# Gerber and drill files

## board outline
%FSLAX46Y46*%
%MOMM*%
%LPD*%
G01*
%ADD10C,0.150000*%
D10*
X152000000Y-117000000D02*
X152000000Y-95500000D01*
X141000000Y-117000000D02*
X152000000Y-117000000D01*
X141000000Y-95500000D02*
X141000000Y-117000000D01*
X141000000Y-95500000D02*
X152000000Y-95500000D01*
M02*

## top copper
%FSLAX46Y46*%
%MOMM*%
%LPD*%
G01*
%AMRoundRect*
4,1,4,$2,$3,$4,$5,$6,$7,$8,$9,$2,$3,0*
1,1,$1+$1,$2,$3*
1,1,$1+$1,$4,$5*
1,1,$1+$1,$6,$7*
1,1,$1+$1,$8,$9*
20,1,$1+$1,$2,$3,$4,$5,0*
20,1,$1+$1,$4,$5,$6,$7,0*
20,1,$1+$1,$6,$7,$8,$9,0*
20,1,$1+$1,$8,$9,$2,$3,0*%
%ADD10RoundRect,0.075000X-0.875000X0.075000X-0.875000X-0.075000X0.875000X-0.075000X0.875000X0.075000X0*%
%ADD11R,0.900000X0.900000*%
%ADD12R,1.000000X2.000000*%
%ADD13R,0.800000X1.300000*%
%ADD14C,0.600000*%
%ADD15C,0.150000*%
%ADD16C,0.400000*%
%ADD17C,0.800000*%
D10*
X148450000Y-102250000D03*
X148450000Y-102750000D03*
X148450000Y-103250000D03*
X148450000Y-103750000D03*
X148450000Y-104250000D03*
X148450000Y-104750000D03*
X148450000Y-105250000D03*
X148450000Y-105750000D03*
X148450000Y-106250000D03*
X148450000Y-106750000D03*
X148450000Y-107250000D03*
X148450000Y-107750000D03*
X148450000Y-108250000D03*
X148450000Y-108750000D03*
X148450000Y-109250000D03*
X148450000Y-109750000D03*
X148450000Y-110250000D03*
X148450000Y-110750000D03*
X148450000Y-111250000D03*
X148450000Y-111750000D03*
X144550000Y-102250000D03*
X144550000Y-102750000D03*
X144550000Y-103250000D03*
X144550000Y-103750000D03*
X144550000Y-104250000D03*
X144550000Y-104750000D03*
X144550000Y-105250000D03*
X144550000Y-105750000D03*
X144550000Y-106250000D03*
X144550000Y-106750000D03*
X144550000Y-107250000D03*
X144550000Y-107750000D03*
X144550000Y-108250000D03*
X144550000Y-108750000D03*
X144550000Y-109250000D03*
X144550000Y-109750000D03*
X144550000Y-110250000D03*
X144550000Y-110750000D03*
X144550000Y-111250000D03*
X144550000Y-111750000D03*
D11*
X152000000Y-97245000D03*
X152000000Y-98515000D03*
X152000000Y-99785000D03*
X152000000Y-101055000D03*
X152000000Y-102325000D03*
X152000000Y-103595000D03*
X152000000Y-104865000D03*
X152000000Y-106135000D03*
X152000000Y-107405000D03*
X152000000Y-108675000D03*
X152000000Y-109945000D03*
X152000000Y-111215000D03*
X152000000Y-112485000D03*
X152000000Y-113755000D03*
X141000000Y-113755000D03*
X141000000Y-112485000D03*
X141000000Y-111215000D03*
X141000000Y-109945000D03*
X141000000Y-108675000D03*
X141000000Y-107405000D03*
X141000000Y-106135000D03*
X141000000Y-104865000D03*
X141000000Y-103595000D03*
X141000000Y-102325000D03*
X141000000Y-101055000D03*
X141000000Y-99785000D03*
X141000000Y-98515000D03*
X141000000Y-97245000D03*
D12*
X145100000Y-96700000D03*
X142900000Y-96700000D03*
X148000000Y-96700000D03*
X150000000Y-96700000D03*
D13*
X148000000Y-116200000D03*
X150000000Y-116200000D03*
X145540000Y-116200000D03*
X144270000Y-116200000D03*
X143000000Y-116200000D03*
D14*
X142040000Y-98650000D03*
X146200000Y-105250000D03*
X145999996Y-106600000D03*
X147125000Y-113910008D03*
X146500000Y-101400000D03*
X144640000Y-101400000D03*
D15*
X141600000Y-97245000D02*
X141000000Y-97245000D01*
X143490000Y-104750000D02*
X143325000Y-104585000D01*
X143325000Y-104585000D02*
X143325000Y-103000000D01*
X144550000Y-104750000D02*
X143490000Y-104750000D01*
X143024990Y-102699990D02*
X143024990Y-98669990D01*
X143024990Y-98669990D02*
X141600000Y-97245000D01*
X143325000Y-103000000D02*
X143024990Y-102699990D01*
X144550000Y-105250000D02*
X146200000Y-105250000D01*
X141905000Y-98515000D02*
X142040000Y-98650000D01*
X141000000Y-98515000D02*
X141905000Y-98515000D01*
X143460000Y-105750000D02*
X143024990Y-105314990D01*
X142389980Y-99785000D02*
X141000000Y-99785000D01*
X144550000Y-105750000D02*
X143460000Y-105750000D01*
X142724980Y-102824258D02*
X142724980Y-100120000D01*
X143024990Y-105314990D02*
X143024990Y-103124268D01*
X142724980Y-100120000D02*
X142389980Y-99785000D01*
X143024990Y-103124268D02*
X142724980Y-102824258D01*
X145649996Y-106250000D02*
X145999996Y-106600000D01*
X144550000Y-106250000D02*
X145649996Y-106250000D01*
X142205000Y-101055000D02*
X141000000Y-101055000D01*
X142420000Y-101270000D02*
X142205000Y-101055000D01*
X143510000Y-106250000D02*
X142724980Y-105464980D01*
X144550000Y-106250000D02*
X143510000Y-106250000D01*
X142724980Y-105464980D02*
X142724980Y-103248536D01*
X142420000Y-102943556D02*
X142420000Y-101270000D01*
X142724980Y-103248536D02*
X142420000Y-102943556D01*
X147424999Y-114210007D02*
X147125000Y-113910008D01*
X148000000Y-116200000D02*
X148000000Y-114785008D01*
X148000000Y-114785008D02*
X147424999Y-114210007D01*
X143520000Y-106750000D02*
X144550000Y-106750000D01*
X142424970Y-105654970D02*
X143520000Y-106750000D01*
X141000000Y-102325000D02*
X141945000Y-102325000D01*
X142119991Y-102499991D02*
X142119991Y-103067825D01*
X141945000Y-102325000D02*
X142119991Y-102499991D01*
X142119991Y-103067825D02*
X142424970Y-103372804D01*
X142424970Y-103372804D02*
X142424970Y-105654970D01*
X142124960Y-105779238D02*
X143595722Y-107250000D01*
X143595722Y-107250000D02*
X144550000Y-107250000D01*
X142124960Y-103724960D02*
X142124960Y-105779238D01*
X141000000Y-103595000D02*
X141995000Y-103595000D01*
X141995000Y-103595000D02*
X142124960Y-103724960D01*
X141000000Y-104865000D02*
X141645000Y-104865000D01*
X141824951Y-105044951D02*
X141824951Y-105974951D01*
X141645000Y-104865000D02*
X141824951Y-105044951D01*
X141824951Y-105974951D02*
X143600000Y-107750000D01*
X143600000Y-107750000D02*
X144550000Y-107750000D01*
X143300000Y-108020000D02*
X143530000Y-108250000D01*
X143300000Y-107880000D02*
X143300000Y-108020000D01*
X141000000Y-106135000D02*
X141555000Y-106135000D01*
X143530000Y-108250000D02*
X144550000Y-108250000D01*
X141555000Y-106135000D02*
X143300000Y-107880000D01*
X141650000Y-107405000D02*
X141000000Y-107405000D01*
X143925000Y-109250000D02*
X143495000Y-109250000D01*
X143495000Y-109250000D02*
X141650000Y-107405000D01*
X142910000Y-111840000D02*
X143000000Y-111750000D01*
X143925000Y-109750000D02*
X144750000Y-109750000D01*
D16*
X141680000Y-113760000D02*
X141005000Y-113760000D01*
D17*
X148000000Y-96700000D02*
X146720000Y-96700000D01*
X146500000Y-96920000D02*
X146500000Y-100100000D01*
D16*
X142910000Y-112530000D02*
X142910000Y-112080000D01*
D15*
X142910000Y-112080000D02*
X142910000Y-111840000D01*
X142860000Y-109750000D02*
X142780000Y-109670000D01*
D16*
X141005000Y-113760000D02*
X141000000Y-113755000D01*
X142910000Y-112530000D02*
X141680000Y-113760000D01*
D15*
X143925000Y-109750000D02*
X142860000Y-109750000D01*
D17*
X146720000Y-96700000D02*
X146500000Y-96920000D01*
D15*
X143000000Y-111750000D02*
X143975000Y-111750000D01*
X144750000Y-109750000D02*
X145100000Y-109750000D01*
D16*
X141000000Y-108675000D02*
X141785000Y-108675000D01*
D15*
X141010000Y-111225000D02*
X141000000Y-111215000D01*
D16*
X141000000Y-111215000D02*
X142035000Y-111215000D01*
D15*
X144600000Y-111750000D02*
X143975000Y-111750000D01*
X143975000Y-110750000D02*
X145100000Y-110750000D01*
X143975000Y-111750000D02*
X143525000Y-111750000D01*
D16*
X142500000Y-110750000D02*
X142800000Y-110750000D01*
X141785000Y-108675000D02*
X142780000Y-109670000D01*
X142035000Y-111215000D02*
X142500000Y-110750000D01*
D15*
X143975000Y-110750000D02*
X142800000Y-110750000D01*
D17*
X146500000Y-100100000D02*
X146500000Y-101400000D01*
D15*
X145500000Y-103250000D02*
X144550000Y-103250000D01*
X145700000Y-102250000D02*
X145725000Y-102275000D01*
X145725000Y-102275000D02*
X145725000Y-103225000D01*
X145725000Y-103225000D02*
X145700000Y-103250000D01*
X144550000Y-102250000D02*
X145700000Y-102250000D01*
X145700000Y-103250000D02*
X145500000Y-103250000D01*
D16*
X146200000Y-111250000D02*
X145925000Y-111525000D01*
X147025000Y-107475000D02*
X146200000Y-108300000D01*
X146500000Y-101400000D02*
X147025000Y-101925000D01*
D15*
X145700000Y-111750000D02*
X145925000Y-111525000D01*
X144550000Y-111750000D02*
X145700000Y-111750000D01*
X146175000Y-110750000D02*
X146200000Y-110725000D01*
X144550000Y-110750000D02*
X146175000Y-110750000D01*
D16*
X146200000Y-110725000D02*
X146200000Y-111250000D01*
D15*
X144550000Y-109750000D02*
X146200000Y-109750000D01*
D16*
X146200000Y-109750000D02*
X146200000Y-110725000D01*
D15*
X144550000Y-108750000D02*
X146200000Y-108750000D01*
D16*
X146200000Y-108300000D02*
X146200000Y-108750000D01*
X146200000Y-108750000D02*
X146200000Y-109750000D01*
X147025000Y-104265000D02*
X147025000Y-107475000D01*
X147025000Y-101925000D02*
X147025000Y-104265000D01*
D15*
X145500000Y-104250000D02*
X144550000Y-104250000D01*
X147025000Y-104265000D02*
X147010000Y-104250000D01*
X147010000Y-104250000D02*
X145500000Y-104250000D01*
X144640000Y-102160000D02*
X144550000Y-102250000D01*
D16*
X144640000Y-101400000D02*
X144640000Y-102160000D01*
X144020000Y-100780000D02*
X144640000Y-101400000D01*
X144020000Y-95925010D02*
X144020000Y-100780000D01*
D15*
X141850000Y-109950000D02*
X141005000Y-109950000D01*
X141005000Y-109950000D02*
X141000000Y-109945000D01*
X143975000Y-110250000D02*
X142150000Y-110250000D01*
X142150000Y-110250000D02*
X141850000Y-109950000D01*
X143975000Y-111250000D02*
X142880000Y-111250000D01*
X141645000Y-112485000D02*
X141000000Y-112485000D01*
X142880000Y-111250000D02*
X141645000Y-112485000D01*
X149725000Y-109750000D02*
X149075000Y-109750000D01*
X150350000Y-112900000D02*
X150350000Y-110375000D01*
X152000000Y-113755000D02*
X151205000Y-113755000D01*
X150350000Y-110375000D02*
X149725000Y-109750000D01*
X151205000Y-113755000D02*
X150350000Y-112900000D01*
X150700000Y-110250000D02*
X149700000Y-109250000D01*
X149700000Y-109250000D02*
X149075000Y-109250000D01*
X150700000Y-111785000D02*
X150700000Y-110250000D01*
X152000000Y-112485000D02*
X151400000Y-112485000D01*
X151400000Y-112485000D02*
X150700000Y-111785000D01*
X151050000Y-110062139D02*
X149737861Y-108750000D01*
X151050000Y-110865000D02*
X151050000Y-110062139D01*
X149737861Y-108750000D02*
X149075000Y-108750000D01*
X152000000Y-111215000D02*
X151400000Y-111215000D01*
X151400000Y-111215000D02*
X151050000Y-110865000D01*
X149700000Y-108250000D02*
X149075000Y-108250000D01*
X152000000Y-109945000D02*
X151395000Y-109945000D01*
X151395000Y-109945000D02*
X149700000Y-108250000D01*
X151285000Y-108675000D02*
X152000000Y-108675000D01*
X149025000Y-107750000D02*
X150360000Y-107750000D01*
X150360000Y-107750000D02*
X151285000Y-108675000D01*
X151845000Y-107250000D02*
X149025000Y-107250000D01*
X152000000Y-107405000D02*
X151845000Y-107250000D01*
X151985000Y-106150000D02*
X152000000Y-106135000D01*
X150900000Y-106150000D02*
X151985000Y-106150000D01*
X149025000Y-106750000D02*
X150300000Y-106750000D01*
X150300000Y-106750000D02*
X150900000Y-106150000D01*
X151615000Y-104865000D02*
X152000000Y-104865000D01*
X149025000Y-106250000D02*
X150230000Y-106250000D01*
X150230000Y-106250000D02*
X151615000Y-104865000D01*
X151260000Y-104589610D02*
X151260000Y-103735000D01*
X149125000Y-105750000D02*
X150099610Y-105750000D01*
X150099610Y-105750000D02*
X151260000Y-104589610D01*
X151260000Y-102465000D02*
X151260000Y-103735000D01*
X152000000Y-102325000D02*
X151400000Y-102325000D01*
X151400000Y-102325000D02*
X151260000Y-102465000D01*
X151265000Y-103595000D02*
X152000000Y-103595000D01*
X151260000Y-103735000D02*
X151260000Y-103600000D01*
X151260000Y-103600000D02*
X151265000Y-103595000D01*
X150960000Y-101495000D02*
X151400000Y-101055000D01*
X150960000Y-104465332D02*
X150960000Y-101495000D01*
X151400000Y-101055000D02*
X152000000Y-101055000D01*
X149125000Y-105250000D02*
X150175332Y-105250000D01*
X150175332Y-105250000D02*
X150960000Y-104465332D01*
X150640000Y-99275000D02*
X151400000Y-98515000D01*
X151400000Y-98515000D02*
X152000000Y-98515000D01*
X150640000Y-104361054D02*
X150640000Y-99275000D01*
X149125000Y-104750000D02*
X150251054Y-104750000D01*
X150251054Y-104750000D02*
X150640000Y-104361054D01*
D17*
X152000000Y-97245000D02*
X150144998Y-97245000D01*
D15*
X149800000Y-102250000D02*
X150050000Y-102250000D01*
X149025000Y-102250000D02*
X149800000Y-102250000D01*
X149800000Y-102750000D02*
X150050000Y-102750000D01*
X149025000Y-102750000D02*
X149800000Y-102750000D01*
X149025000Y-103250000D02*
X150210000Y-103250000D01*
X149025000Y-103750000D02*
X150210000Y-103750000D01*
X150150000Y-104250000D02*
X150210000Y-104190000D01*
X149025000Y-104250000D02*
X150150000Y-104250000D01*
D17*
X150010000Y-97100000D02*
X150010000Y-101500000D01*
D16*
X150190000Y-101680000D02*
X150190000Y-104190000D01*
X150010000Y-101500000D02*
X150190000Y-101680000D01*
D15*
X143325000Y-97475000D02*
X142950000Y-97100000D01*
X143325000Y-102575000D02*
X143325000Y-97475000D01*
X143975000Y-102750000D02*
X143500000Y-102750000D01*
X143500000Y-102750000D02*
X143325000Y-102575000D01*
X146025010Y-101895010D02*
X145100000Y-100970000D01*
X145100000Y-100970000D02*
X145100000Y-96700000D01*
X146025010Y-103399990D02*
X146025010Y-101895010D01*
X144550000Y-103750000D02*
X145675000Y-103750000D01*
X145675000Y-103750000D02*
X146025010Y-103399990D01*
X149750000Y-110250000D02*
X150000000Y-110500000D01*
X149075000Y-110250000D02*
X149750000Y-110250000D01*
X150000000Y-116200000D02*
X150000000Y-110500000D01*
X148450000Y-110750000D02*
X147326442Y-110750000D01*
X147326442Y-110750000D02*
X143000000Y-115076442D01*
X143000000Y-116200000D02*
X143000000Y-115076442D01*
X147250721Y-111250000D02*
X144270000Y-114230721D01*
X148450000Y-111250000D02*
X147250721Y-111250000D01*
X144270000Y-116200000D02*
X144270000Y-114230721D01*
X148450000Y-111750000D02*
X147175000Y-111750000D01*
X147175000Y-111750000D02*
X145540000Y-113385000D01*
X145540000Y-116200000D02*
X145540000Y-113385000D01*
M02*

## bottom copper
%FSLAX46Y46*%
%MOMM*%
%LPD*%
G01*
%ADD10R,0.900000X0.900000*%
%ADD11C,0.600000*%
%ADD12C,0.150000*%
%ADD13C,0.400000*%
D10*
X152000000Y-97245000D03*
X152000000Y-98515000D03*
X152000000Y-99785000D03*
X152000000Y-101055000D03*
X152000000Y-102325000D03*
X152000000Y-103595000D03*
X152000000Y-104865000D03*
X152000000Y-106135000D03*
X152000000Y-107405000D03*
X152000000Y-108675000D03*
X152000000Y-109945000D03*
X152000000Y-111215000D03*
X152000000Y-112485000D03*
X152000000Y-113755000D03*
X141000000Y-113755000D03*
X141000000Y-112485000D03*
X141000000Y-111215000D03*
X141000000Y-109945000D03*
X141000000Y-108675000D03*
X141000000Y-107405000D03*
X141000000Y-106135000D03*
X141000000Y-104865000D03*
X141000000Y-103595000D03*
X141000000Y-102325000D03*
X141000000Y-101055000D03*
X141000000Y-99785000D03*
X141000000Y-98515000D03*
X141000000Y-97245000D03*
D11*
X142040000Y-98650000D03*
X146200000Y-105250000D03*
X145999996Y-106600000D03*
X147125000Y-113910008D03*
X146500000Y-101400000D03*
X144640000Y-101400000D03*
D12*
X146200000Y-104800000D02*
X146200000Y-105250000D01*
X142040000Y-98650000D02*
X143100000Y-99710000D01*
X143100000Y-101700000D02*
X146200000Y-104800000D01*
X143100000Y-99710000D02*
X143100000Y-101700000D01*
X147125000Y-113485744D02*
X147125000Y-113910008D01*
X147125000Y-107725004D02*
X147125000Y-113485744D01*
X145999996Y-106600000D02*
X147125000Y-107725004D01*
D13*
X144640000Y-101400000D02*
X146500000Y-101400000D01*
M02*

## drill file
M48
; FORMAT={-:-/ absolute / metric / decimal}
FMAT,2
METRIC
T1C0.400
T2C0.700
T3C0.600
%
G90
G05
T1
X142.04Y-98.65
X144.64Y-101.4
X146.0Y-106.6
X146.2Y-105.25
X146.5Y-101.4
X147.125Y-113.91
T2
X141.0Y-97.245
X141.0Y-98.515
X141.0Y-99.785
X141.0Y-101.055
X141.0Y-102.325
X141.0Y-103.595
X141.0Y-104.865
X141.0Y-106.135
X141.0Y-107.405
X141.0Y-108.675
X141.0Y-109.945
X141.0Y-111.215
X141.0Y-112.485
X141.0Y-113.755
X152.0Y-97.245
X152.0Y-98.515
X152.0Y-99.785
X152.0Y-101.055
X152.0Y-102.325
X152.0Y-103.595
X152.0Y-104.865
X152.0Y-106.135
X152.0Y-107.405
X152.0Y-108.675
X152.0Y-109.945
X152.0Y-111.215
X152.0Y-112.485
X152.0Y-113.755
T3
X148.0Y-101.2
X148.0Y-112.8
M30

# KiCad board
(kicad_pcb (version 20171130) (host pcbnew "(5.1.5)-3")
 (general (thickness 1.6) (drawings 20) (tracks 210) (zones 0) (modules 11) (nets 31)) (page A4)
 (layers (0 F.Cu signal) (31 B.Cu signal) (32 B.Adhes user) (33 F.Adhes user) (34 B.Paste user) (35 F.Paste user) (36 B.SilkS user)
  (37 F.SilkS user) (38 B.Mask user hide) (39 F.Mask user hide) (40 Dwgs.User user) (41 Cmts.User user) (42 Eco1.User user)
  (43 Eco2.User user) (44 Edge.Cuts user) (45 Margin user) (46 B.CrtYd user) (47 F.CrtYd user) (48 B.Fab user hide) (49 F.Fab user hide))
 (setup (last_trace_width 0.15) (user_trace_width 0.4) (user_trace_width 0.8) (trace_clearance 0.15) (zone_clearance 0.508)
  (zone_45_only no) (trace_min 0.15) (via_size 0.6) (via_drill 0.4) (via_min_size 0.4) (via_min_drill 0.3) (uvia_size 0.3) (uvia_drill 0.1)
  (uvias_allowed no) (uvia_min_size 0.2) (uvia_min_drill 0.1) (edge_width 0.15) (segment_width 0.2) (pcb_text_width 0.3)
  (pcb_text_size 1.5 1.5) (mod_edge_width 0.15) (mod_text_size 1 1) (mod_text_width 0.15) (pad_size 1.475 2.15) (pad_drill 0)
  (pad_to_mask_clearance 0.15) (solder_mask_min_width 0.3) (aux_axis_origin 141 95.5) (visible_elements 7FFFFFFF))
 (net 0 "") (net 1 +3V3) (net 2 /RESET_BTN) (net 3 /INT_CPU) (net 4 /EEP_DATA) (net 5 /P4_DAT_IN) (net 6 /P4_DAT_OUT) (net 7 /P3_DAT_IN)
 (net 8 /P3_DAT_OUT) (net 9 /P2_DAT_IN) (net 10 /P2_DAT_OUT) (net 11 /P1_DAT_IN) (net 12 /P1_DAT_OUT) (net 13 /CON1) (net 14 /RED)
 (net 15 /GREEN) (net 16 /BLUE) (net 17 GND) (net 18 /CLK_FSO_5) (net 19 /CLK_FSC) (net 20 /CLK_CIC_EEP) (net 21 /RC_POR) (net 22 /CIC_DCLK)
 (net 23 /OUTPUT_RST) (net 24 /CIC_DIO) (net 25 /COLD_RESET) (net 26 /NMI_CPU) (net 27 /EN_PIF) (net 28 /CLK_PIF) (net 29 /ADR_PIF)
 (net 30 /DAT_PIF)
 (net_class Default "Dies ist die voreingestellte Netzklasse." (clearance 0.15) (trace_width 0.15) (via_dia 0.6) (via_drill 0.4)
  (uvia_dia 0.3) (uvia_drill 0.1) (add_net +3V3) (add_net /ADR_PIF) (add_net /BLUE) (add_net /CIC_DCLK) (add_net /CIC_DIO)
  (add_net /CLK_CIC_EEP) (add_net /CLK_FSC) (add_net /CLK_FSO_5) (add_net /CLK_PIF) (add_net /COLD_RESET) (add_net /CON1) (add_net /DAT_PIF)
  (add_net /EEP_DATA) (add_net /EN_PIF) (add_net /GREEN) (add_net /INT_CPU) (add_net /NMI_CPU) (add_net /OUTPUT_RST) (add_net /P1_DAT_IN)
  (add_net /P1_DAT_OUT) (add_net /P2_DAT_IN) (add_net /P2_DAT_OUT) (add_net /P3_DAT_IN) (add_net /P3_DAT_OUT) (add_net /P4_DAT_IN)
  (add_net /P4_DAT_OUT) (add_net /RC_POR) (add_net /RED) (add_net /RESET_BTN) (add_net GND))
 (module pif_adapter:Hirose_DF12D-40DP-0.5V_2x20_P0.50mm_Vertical (layer F.Cu) (at 146.5 107 270)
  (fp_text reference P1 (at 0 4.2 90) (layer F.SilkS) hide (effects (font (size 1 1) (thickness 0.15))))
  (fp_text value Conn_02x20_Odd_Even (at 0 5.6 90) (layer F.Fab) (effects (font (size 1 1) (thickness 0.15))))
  (pad 2 smd roundrect (at -4.75 -1.95 270) (size 0.3 1.9) (layers F.Cu F.Mask) (roundrect_rratio 0.25) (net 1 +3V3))
  (pad 4 smd roundrect (at -4.25 -1.95 270) (size 0.3 1.9) (layers F.Cu F.Mask) (roundrect_rratio 0.25) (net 1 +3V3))
  (pad 6 smd roundrect (at -3.75 -1.95 270) (size 0.3 1.9) (layers F.Cu F.Mask) (roundrect_rratio 0.25) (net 1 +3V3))
  (pad 8 smd roundrect (at -3.25 -1.95 270) (size 0.3 1.9) (layers F.Cu F.Mask) (roundrect_rratio 0.25) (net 1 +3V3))
  (pad 10 smd roundrect (at -2.75 -1.95 270) (size 0.3 1.9) (layers F.Cu F.Mask) (roundrect_rratio 0.25) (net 1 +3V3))
  (pad 12 smd roundrect (at -2.25 -1.95 270) (size 0.3 1.9) (layers F.Cu F.Mask) (roundrect_rratio 0.25) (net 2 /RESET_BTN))
  (pad 14 smd roundrect (at -1.75 -1.95 270) (size 0.3 1.9) (layers F.Cu F.Mask) (roundrect_rratio 0.25) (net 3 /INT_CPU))
  (pad 16 smd roundrect (at -1.25 -1.95 270) (size 0.3 1.9) (layers F.Cu F.Mask) (roundrect_rratio 0.25) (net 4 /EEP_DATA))
  (pad 18 smd roundrect (at -0.75 -1.95 270) (size 0.3 1.9) (layers F.Cu F.Mask) (roundrect_rratio 0.25) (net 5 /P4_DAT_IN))
  (pad 20 smd roundrect (at -0.25 -1.95 270) (size 0.3 1.9) (layers F.Cu F.Mask) (roundrect_rratio 0.25) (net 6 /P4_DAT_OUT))
  (pad 22 smd roundrect (at 0.25 -1.95 270) (size 0.3 1.9) (layers F.Cu F.Mask) (roundrect_rratio 0.25) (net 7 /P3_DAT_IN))
  (pad 24 smd roundrect (at 0.75 -1.95 270) (size 0.3 1.9) (layers F.Cu F.Mask) (roundrect_rratio 0.25) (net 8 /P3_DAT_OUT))
  (pad 26 smd roundrect (at 1.25 -1.95 270) (size 0.3 1.9) (layers F.Cu F.Mask) (roundrect_rratio 0.25) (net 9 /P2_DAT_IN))
  (pad 28 smd roundrect (at 1.75 -1.95 270) (size 0.3 1.9) (layers F.Cu F.Mask) (roundrect_rratio 0.25) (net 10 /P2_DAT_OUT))
  (pad 30 smd roundrect (at 2.25 -1.95 270) (size 0.3 1.9) (layers F.Cu F.Mask) (roundrect_rratio 0.25) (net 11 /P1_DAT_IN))
  (pad 32 smd roundrect (at 2.75 -1.95 270) (size 0.3 1.9) (layers F.Cu F.Mask) (roundrect_rratio 0.25) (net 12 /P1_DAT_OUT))
  (pad 34 smd roundrect (at 3.25 -1.95 270) (size 0.3 1.9) (layers F.Cu F.Mask) (roundrect_rratio 0.25) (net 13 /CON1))
  (pad 36 smd roundrect (at 3.75 -1.95 270) (size 0.3 1.9) (layers F.Cu F.Mask) (roundrect_rratio 0.25) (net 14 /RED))
  (pad 38 smd roundrect (at 4.25 -1.95 270) (size 0.3 1.9) (layers F.Cu F.Mask) (roundrect_rratio 0.25) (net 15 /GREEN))
  (pad 40 smd roundrect (at 4.75 -1.95 270) (size 0.3 1.9) (layers F.Cu F.Mask) (roundrect_rratio 0.25) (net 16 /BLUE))
  (pad 1 smd roundrect (at -4.75 1.95 270) (size 0.3 1.9) (layers F.Cu F.Mask) (roundrect_rratio 0.25) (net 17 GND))
  (pad 3 smd roundrect (at -4.25 1.95 270) (size 0.3 1.9) (layers F.Cu F.Mask) (roundrect_rratio 0.25) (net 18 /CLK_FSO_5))
  (pad 5 smd roundrect (at -3.75 1.95 270) (size 0.3 1.9) (layers F.Cu F.Mask) (roundrect_rratio 0.25) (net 17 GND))
  (pad 7 smd roundrect (at -3.25 1.95 270) (size 0.3 1.9) (layers F.Cu F.Mask) (roundrect_rratio 0.25) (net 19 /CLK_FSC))
  (pad 9 smd roundrect (at -2.75 1.95 270) (size 0.3 1.9) (layers F.Cu F.Mask) (roundrect_rratio 0.25) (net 17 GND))
  (pad 11 smd roundrect (at -2.25 1.95 270) (size 0.3 1.9) (layers F.Cu F.Mask) (roundrect_rratio 0.25) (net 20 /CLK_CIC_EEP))
  (pad 13 smd roundrect (at -1.75 1.95 270) (size 0.3 1.9) (layers F.Cu F.Mask) (roundrect_rratio 0.25) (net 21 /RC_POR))
  (pad 15 smd roundrect (at -1.25 1.95 270) (size 0.3 1.9) (layers F.Cu F.Mask) (roundrect_rratio 0.25) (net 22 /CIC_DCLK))
  (pad 17 smd roundrect (at -0.75 1.95 270) (size 0.3 1.9) (layers F.Cu F.Mask) (roundrect_rratio 0.25) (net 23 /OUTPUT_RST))
  (pad 19 smd roundrect (at -0.25 1.95 270) (size 0.3 1.9) (layers F.Cu F.Mask) (roundrect_rratio 0.25) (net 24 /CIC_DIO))
  (pad 21 smd roundrect (at 0.25 1.95 270) (size 0.3 1.9) (layers F.Cu F.Mask) (roundrect_rratio 0.25) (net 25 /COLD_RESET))
  (pad 23 smd roundrect (at 0.75 1.95 270) (size 0.3 1.9) (layers F.Cu F.Mask) (roundrect_rratio 0.25) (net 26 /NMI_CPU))
  (pad 25 smd roundrect (at 1.25 1.95 270) (size 0.3 1.9) (layers F.Cu F.Mask) (roundrect_rratio 0.25) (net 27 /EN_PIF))
  (pad 27 smd roundrect (at 1.75 1.95 270) (size 0.3 1.9) (layers F.Cu F.Mask) (roundrect_rratio 0.25) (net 17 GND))
  (pad 29 smd roundrect (at 2.25 1.95 270) (size 0.3 1.9) (layers F.Cu F.Mask) (roundrect_rratio 0.25) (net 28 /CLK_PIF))
  (pad 31 smd roundrect (at 2.75 1.95 270) (size 0.3 1.9) (layers F.Cu F.Mask) (roundrect_rratio 0.25) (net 17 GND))
  (pad 33 smd roundrect (at 3.25 1.95 270) (size 0.3 1.9) (layers F.Cu F.Mask) (roundrect_rratio 0.25) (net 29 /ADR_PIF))
  (pad 35 smd roundrect (at 3.75 1.95 270) (size 0.3 1.9) (layers F.Cu F.Mask) (roundrect_rratio 0.25) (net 17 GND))
  (pad 37 smd roundrect (at 4.25 1.95 270) (size 0.3 1.9) (layers F.Cu F.Mask) (roundrect_rratio 0.25) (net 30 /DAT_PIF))
  (pad 39 smd roundrect (at 4.75 1.95 270) (size 0.3 1.9) (layers F.Cu F.Mask) (roundrect_rratio 0.25) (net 17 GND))
  (pad "" smd rect (at -4.75 -2 270) (size 0.28 1.2) (layers F.Paste))
  (pad "" smd rect (at -4.25 -2 270) (size 0.28 1.2) (layers F.Paste))
  (pad "" smd rect (at -3.75 -2 270) (size 0.28 1.2) (layers F.Paste))
  (pad "" smd rect (at -3.25 -2 270) (size 0.28 1.2) (layers F.Paste))
  (pad "" smd rect (at -2.75 -2 270) (size 0.28 1.2) (layers F.Paste))
  (pad "" smd rect (at -2.25 -2 270) (size 0.28 1.2) (layers F.Paste))
  (pad "" smd rect (at -1.75 -2 270) (size 0.28 1.2) (layers F.Paste))
  (pad "" smd rect (at -1.25 -2 270) (size 0.28 1.2) (layers F.Paste))
  (pad "" smd rect (at -0.75 -2 270) (size 0.28 1.2) (layers F.Paste))
  (pad "" smd rect (at -0.25 -2 270) (size 0.28 1.2) (layers F.Paste))
  (pad "" smd rect (at 0.25 -2 270) (size 0.28 1.2) (layers F.Paste))
  (pad "" smd rect (at 0.75 -2 270) (size 0.28 1.2) (layers F.Paste))
  (pad "" smd rect (at 1.25 -2 270) (size 0.28 1.2) (layers F.Paste))
  (pad "" smd rect (at 1.75 -2 270) (size 0.28 1.2) (layers F.Paste))
  (pad "" smd rect (at 2.25 -2 270) (size 0.28 1.2) (layers F.Paste))
  (pad "" smd rect (at 2.75 -2 270) (size 0.28 1.2) (layers F.Paste))
  (pad "" smd rect (at 3.25 -2 270) (size 0.28 1.2) (layers F.Paste))
  (pad "" smd rect (at 3.75 -2 270) (size 0.28 1.2) (layers F.Paste))
  (pad "" smd rect (at 4.25 -2 270) (size 0.28 1.2) (layers F.Paste))
  (pad "" smd rect (at 4.75 -2 270) (size 0.28 1.2) (layers F.Paste))
  (pad "" smd rect (at -4.75 2 270) (size 0.28 1.2) (layers F.Paste))
  (pad "" smd rect (at -4.25 2 270) (size 0.28 1.2) (layers F.Paste))
  (pad "" smd rect (at -3.75 2 270) (size 0.28 1.2) (layers F.Paste))
  (pad "" smd rect (at -3.25 2 270) (size 0.28 1.2) (layers F.Paste))
  (pad "" smd rect (at -2.75 2 270) (size 0.28 1.2) (layers F.Paste))
  (pad "" smd rect (at -2.25 2 270) (size 0.28 1.2) (layers F.Paste))
  (pad "" smd rect (at -1.75 2 270) (size 0.28 1.2) (layers F.Paste))
  (pad "" smd rect (at -1.25 2 270) (size 0.28 1.2) (layers F.Paste))
  (pad "" smd rect (at -0.75 2 270) (size 0.28 1.2) (layers F.Paste))
  (pad "" smd rect (at -0.25 2 270) (size 0.28 1.2) (layers F.Paste))
  (pad "" smd rect (at 0.25 2 270) (size 0.28 1.2) (layers F.Paste))
  (pad "" smd rect (at 0.75 2 270) (size 0.28 1.2) (layers F.Paste))
  (pad "" smd rect (at 1.25 2 270) (size 0.28 1.2) (layers F.Paste))
  (pad "" smd rect (at 1.75 2 270) (size 0.28 1.2) (layers F.Paste))
  (pad "" smd rect (at 2.25 2 270) (size 0.28 1.2) (layers F.Paste))
  (pad "" smd rect (at 2.75 2 270) (size 0.28 1.2) (layers F.Paste))
  (pad "" smd rect (at 3.25 2 270) (size 0.28 1.2) (layers F.Paste))
  (pad "" smd rect (at 3.75 2 270) (size 0.28 1.2) (layers F.Paste))
  (pad "" smd rect (at 4.25 2 270) (size 0.28 1.2) (layers F.Paste))
  (pad "" smd rect (at 4.75 2 270) (size 0.28 1.2) (layers F.Paste))
  (pad "" np_thru_hole circle (at -5.8 -1.5 270) (size 0.6 0.6) (drill 0.6) (layers *.Cu *.Mask))
  (pad "" np_thru_hole circle (at 5.8 -1.5 270) (size 0.6 0.6) (drill 0.6) (layers *.Cu *.Mask)))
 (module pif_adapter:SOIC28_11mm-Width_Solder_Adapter (layer F.Cu) (at 146.5 105.5 270)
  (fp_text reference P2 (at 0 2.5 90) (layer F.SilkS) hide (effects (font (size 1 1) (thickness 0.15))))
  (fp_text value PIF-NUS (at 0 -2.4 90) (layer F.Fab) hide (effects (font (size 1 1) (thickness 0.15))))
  (pad 28 thru_hole rect (at -8.255 -5.5 270) (size 0.9 0.9) (drill 0.7) (layers *.Cu *.Mask) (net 1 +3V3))
  (pad 27 thru_hole rect (at -6.985 -5.5 270) (size 0.9 0.9) (drill 0.7) (layers *.Cu *.Mask) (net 2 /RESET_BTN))
  (pad 26 thru_hole rect (at -5.715 -5.5 270) (size 0.9 0.9) (drill 0.7) (layers *.Cu *.Mask))
  (pad 25 thru_hole rect (at -4.445 -5.5 270) (size 0.9 0.9) (drill 0.7) (layers *.Cu *.Mask) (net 3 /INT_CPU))
  (pad 24 thru_hole rect (at -3.175 -5.5 270) (size 0.9 0.9) (drill 0.7) (layers *.Cu *.Mask) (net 4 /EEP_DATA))
  (pad 23 thru_hole rect (at -1.905 -5.5 270) (size 0.9 0.9) (drill 0.7) (layers *.Cu *.Mask) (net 4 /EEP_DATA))
  (pad 22 thru_hole rect (at -0.635 -5.5 270) (size 0.9 0.9) (drill 0.7) (layers *.Cu *.Mask) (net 5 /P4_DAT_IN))
  (pad 21 thru_hole rect (at 0.635 -5.5 270) (size 0.9 0.9) (drill 0.7) (layers *.Cu *.Mask) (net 6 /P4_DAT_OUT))
  (pad 20 thru_hole rect (at 1.905 -5.5 270) (size 0.9 0.9) (drill 0.7) (layers *.Cu *.Mask) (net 7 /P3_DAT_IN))
  (pad 19 thru_hole rect (at 3.175 -5.5 270) (size 0.9 0.9) (drill 0.7) (layers *.Cu *.Mask) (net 8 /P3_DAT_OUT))
  (pad 18 thru_hole rect (at 4.445 -5.5 270) (size 0.9 0.9) (drill 0.7) (layers *.Cu *.Mask) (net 9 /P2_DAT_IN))
  (pad 17 thru_hole rect (at 5.715 -5.5 270) (size 0.9 0.9) (drill 0.7) (layers *.Cu *.Mask) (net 10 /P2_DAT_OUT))
  (pad 16 thru_hole rect (at 6.985 -5.5 270) (size 0.9 0.9) (drill 0.7) (layers *.Cu *.Mask) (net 11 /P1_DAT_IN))
  (pad 15 thru_hole rect (at 8.255 -5.5 270) (size 0.9 0.9) (drill 0.7) (layers *.Cu *.Mask) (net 12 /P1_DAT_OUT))
  (pad 14 thru_hole rect (at 8.255 5.5 270) (size 0.9 0.9) (drill 0.7) (layers *.Cu *.Mask) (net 17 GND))
  (pad 13 thru_hole rect (at 6.985 5.5 270) (size 0.9 0.9) (drill 0.7) (layers *.Cu *.Mask) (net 30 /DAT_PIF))
  (pad 12 thru_hole rect (at 5.715 5.5 270) (size 0.9 0.9) (drill 0.7) (layers *.Cu *.Mask) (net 17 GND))
  (pad 11 thru_hole rect (at 4.445 5.5 270) (size 0.9 0.9) (drill 0.7) (layers *.Cu *.Mask) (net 29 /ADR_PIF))
  (pad 10 thru_hole rect (at 3.175 5.5 270) (size 0.9 0.9) (drill 0.7) (layers *.Cu *.Mask) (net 17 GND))
  (pad 9 thru_hole rect (at 1.905 5.5 270) (size 0.9 0.9) (drill 0.7) (layers *.Cu *.Mask) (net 28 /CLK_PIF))
  (pad 8 thru_hole rect (at 0.635 5.5 270) (size 0.9 0.9) (drill 0.7) (layers *.Cu *.Mask) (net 27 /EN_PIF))
  (pad 7 thru_hole rect (at -0.635 5.5 270) (size 0.9 0.9) (drill 0.7) (layers *.Cu *.Mask) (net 26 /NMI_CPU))
  (pad 6 thru_hole rect (at -1.905 5.5 270) (size 0.9 0.9) (drill 0.7) (layers *.Cu *.Mask) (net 25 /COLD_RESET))
  (pad 5 thru_hole rect (at -3.175 5.5 270) (size 0.9 0.9) (drill 0.7) (layers *.Cu *.Mask) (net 24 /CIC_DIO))
  (pad 4 thru_hole rect (at -4.445 5.5 270) (size 0.9 0.9) (drill 0.7) (layers *.Cu *.Mask) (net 23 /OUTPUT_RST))
  (pad 3 thru_hole rect (at -5.715 5.5 270) (size 0.9 0.9) (drill 0.7) (layers *.Cu *.Mask) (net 22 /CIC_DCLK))
  (pad 2 thru_hole rect (at -6.985 5.5 270) (size 0.9 0.9) (drill 0.7) (layers *.Cu *.Mask) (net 21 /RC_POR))
  (pad 1 thru_hole rect (at -8.255 5.5 270) (size 0.9 0.9) (drill 0.7) (layers *.Cu *.Mask) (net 20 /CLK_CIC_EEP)))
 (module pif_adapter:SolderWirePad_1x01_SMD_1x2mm (layer F.Cu) (at 145.1 96.7)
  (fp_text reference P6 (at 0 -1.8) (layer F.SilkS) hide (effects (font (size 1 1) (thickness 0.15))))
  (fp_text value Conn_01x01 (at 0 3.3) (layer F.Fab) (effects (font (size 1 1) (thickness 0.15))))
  (pad 1 smd rect (at 0 0) (size 1 2) (layers F.Cu F.Paste F.Mask) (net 19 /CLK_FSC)))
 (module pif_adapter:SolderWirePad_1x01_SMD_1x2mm (layer F.Cu) (at 142.9 96.7)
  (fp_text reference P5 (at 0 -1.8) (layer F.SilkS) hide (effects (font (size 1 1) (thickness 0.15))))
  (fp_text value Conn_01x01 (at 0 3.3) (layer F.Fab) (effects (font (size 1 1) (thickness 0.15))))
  (pad 1 smd rect (at 0 0) (size 1 2) (layers F.Cu F.Paste F.Mask) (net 18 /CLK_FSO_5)))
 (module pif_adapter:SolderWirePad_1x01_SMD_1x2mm (layer F.Cu) (at 148 96.7)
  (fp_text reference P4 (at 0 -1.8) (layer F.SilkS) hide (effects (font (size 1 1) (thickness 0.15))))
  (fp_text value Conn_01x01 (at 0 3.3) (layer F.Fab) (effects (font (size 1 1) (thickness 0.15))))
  (pad 1 smd rect (at 0 0) (size 1 2) (layers F.Cu F.Paste F.Mask) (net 17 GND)))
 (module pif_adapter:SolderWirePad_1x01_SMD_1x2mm (layer F.Cu) (at 150 96.7)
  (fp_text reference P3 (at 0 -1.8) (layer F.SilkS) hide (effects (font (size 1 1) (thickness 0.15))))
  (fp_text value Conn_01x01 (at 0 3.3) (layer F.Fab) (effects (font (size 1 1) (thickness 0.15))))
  (pad 1 smd rect (at 0 0) (size 1 2) (layers F.Cu F.Paste F.Mask) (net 1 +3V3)))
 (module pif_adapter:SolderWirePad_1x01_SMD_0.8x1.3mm (layer F.Cu) (at 148 116.2)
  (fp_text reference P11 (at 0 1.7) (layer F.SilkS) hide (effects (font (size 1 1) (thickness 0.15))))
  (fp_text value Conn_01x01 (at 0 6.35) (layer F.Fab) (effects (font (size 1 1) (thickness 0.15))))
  (pad 1 smd rect (at 0 0) (size 0.8 1.3) (layers F.Cu F.Paste F.Mask) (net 23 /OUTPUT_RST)))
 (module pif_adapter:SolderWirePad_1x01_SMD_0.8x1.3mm (layer F.Cu) (at 150 116.2)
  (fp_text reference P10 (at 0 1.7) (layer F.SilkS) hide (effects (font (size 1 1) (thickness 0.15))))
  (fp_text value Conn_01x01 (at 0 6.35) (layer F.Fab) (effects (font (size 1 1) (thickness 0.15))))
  (pad 1 smd rect (at 0 0) (size 0.8 1.3) (layers F.Cu F.Paste F.Mask) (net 13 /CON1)))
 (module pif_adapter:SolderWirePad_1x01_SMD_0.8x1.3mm (layer F.Cu) (at 145.54 116.2)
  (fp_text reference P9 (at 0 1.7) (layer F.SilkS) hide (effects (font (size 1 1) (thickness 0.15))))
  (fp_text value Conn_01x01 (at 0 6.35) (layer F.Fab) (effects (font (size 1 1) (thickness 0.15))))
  (pad 1 smd rect (at 0 0) (size 0.8 1.3) (layers F.Cu F.Paste F.Mask) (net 16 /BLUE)))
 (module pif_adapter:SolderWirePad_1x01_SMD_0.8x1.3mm (layer F.Cu) (at 144.27 116.2)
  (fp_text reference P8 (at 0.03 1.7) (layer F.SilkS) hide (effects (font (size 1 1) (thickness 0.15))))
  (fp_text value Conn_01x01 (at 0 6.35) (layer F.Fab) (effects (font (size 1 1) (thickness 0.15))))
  (pad 1 smd rect (at 0 0) (size 0.8 1.3) (layers F.Cu F.Paste F.Mask) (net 15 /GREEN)))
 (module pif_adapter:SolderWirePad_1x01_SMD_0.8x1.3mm (layer F.Cu) (at 143 116.2)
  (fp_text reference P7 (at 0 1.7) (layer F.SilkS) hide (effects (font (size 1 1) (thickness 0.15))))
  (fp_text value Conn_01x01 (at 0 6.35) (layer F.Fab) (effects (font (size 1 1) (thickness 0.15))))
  (pad 1 smd rect (at 0 0) (size 0.8 1.3) (layers F.Cu F.Paste F.Mask) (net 14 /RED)))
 (gr_line (start 152 117) (end 152 95.5) (layer Edge.Cuts) (width 0.15))
 (gr_line (start 141 117) (end 152 117) (layer Edge.Cuts) (width 0.15))
 (gr_line (start 141 95.5) (end 141 117) (layer Edge.Cuts) (width 0.15))
 (gr_line (start 141 95.5) (end 152 95.5) (layer Edge.Cuts) (width 0.15))
 (segment (start 141.6 97.245) (end 141 97.245) (width 0.15) (layer F.Cu) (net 20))
 (segment (start 143.49 104.75) (end 143.325 104.585) (width 0.15) (layer F.Cu) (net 20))
 (segment (start 143.325 104.585) (end 143.325 103) (width 0.15) (layer F.Cu) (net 20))
 (segment (start 144.55 104.75) (end 143.49 104.75) (width 0.15) (layer F.Cu) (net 20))
 (segment (start 143.02499 102.69999) (end 143.02499 98.66999) (width 0.15) (layer F.Cu) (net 20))
 (segment (start 143.02499 98.66999) (end 141.6 97.245) (width 0.15) (layer F.Cu) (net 20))
 (segment (start 143.325 103) (end 143.02499 102.69999) (width 0.15) (layer F.Cu) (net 20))
 (via (at 142.04 98.65) (size 0.6) (drill 0.4) (layers F.Cu B.Cu) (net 21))
 (via (at 146.2 105.25) (size 0.6) (drill 0.4) (layers F.Cu B.Cu) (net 21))
 (segment (start 144.55 105.25) (end 146.2 105.25) (width 0.15) (layer F.Cu) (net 21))
 (segment (start 141.905 98.515) (end 142.04 98.65) (width 0.15) (layer F.Cu) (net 21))
 (segment (start 141 98.515) (end 141.905 98.515) (width 0.15) (layer F.Cu) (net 21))
 (segment (start 146.2 104.8) (end 146.2 105.25) (width 0.15) (layer B.Cu) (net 21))
 (segment (start 142.04 98.65) (end 143.1 99.71) (width 0.15) (layer B.Cu) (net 21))
 (segment (start 143.1 101.7) (end 146.2 104.8) (width 0.15) (layer B.Cu) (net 21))
 (segment (start 143.1 99.71) (end 143.1 101.7) (width 0.15) (layer B.Cu) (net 21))
 (segment (start 143.46 105.75) (end 143.02499 105.31499) (width 0.15) (layer F.Cu) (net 22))
 (segment (start 142.38998 99.785) (end 141 99.785) (width 0.15) (layer F.Cu) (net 22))
 (segment (start 144.55 105.75) (end 143.46 105.75) (width 0.15) (layer F.Cu) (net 22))
 (segment (start 142.72498 102.824258) (end 142.72498 100.12) (width 0.15) (layer F.Cu) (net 22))
 (segment (start 143.02499 105.31499) (end 143.02499 103.124268) (width 0.15) (layer F.Cu) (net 22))
 (segment (start 142.72498 100.12) (end 142.38998 99.785) (width 0.15) (layer F.Cu) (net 22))
 (segment (start 143.02499 103.124268) (end 142.72498 102.824258) (width 0.15) (layer F.Cu) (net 22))
 (via (at 145.999996 106.6) (size 0.6) (drill 0.4) (layers F.Cu B.Cu) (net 23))
 (segment (start 145.649996 106.25) (end 145.999996 106.6) (width 0.15) (layer F.Cu) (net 23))
 (segment (start 144.55 106.25) (end 145.649996 106.25) (width 0.15) (layer F.Cu) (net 23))
 (segment (start 142.205 101.055) (end 141 101.055) (width 0.15) (layer F.Cu) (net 23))
 (segment (start 142.42 101.27) (end 142.205 101.055) (width 0.15) (layer F.Cu) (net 23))
 (segment (start 143.51 106.25) (end 142.72498 105.46498) (width 0.15) (layer F.Cu) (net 23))
 (segment (start 144.55 106.25) (end 143.51 106.25) (width 0.15) (layer F.Cu) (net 23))
 (segment (start 142.72498 105.46498) (end 142.72498 103.248536) (width 0.15) (layer F.Cu) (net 23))
 (segment (start 142.42 102.943556) (end 142.42 101.27) (width 0.15) (layer F.Cu) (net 23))
 (segment (start 142.72498 103.248536) (end 142.42 102.943556) (width 0.15) (layer F.Cu) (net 23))
 (via (at 147.125 113.910008) (size 0.6) (drill 0.4) (layers F.Cu B.Cu) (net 23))
 (segment (start 147.125 113.485744) (end 147.125 113.910008) (width 0.15) (layer B.Cu) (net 23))
 (segment (start 147.125 107.725004) (end 147.125 113.485744) (width 0.15) (layer B.Cu) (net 23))
 (segment (start 145.999996 106.6) (end 147.125 107.725004) (width 0.15) (layer B.Cu) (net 23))
 (segment (start 147.424999 114.210007) (end 147.125 113.910008) (width 0.15) (layer F.Cu) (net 23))
 (segment (start 148 116.2) (end 148 114.785008) (width 0.15) (layer F.Cu) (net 23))
 (segment (start 148 114.785008) (end 147.424999 114.210007) (width 0.15) (layer F.Cu) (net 23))
 (segment (start 143.52 106.75) (end 144.55 106.75) (width 0.15) (layer F.Cu) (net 24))
 (segment (start 142.42497 105.65497) (end 143.52 106.75) (width 0.15) (layer F.Cu) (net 24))
 (segment (start 141 102.325) (end 141.945 102.325) (width 0.15) (layer F.Cu) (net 24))
 (segment (start 142.119991 102.499991) (end 142.119991 103.067825) (width 0.15) (layer F.Cu) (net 24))
 (segment (start 141.945 102.325) (end 142.119991 102.499991) (width 0.15) (layer F.Cu) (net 24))
 (segment (start 142.119991 103.067825) (end 142.42497 103.372804) (width 0.15) (layer F.Cu) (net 24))
 (segment (start 142.42497 103.372804) (end 142.42497 105.65497) (width 0.15) (layer F.Cu) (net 24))
 (segment (start 142.12496 105.779238) (end 143.595722 107.25) (width 0.15) (layer F.Cu) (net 25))
 (segment (start 143.595722 107.25) (end 144.55 107.25) (width 0.15) (layer F.Cu) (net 25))
 (segment (start 142.12496 103.72496) (end 142.12496 105.779238) (width 0.15) (layer F.Cu) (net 25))
 (segment (start 141 103.595) (end 141.995 103.595) (width 0.15) (layer F.Cu) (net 25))
 (segment (start 141.995 103.595) (end 142.12496 103.72496) (width 0.15) (layer F.Cu) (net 25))
 (segment (start 141 104.865) (end 141.645 104.865) (width 0.15) (layer F.Cu) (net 26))
 (segment (start 141.824951 105.044951) (end 141.824951 105.974951) (width 0.15) (layer F.Cu) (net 26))
 (segment (start 141.645 104.865) (end 141.824951 105.044951) (width 0.15) (layer F.Cu) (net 26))
 (segment (start 141.824951 105.974951) (end 143.6 107.75) (width 0.15) (layer F.Cu) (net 26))
 (segment (start 143.6 107.75) (end 144.55 107.75) (width 0.15) (layer F.Cu) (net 26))
 (segment (start 143.3 108.02) (end 143.53 108.25) (width 0.15) (layer F.Cu) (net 27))
 (segment (start 143.3 107.88) (end 143.3 108.02) (width 0.15) (layer F.Cu) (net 27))
 (segment (start 141 106.135) (end 141.555 106.135) (width 0.15) (layer F.Cu) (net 27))
 (segment (start 143.53 108.25) (end 144.55 108.25) (width 0.15) (layer F.Cu) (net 27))
 (segment (start 141.555 106.135) (end 143.3 107.88) (width 0.15) (layer F.Cu) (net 27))
 (segment (start 141.65 107.405) (end 141 107.405) (width 0.15) (layer F.Cu) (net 28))
 (segment (start 143.925 109.25) (end 143.495 109.25) (width 0.15) (layer F.Cu) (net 28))
 (segment (start 143.495 109.25) (end 141.65 107.405) (width 0.15) (layer F.Cu) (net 28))
 (segment (start 142.91 111.84) (end 143 111.75) (width 0.15) (layer F.Cu) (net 17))
 (segment (start 143.925 109.75) (end 144.75 109.75) (width 0.15) (layer F.Cu) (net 17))
 (segment (start 141.68 113.76) (end 141.005 113.76) (width 0.4) (layer F.Cu) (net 17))
 (segment (start 148 96.7) (end 146.72 96.7) (width 0.8) (layer F.Cu) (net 17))
 (segment (start 146.5 96.92) (end 146.5 100.1) (width 0.8) (layer F.Cu) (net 17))
 (segment (start 142.91 112.53) (end 142.91 112.08) (width 0.4) (layer F.Cu) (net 17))
 (segment (start 142.91 112.08) (end 142.91 111.84) (width 0.15) (layer F.Cu) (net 17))
 (segment (start 142.86 109.75) (end 142.78 109.67) (width 0.15) (layer F.Cu) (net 17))
 (segment (start 141.005 113.76) (end 141 113.755) (width 0.4) (layer F.Cu) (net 17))
 (segment (start 142.91 112.53) (end 141.68 113.76) (width 0.4) (layer F.Cu) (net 17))
 (segment (start 143.925 109.75) (end 142.86 109.75) (width 0.15) (layer F.Cu) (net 17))
 (segment (start 146.72 96.7) (end 146.5 96.92) (width 0.8) (layer F.Cu) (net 17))
 (segment (start 143 111.75) (end 143.975 111.75) (width 0.15) (layer F.Cu) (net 17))
 (segment (start 144.75 109.75) (end 145.1 109.75) (width 0.15) (layer F.Cu) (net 17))
 (segment (start 141 108.675) (end 141.785 108.675) (width 0.4) (layer F.Cu) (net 17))
 (segment (start 141.01 111.225) (end 141 111.215) (width 0.15) (layer F.Cu) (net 17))
 (segment (start 141 111.215) (end 142.035 111.215) (width 0.4) (layer F.Cu) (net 17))
 (segment (start 144.6 111.75) (end 143.975 111.75) (width 0.15) (layer F.Cu) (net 17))
 (segment (start 143.975 110.75) (end 145.1 110.75) (width 0.15) (layer F.Cu) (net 17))
 (segment (start 143.975 111.75) (end 143.525 111.75) (width 0.15) (layer F.Cu) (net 17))
 (segment (start 142.5 110.75) (end 142.8 110.75) (width 0.4) (layer F.Cu) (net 17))
 (segment (start 141.785 108.675) (end 142.78 109.67) (width 0.4) (layer F.Cu) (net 17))
 (segment (start 142.035 111.215) (end 142.5 110.75) (width 0.4) (layer F.Cu) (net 17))
 (segment (start 143.975 110.75) (end 142.8 110.75) (width 0.15) (layer F.Cu) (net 17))
 (segment (start 146.5 100.1) (end 146.5 101.4) (width 0.8) (layer F.Cu) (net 17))
 (via (at 146.5 101.4) (size 0.6) (drill 0.4) (layers F.Cu B.Cu) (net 17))
 (segment (start 145.5 103.25) (end 144.55 103.25) (width 0.15) (layer F.Cu) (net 17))
 (segment (start 145.7 102.25) (end 145.725 102.275) (width 0.15) (layer F.Cu) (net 17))
 (segment (start 145.725 102.275) (end 145.725 103.225) (width 0.15) (layer F.Cu) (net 17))
 (segment (start 145.725 103.225) (end 145.7 103.25) (width 0.15) (layer F.Cu) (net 17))
 (segment (start 144.55 102.25) (end 145.7 102.25) (width 0.15) (layer F.Cu) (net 17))
 (segment (start 145.7 103.25) (end 145.5 103.25) (width 0.15) (layer F.Cu) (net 17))
 (segment (start 146.2 111.25) (end 145.925 111.525) (width 0.4) (layer F.Cu) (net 17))
 (segment (start 147.025 107.475) (end 146.2 108.3) (width 0.4) (layer F.Cu) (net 17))
 (segment (start 146.5 101.4) (end 147.025 101.925) (width 0.4) (layer F.Cu) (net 17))
 (segment (start 145.7 111.75) (end 145.925 111.525) (width 0.15) (layer F.Cu) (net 17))
 (segment (start 144.55 111.75) (end 145.7 111.75) (width 0.15) (layer F.Cu) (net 17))
 (segment (start 146.175 110.75) (end 146.2 110.725) (width 0.15) (layer F.Cu) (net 17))
 (segment (start 144.55 110.75) (end 146.175 110.75) (width 0.15) (layer F.Cu) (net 17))
 (segment (start 146.2 110.725) (end 146.2 111.25) (width 0.4) (layer F.Cu) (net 17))
 (segment (start 144.55 109.75) (end 146.2 109.75) (width 0.15) (layer F.Cu) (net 17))
 (segment (start 146.2 109.75) (end 146.2 110.725) (width 0.4) (layer F.Cu) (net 17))
 (segment (start 144.55 108.75) (end 146.2 108.75) (width 0.15) (layer F.Cu) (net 17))
 (segment (start 146.2 108.3) (end 146.2 108.75) (width 0.4) (layer F.Cu) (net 17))
 (segment (start 146.2 108.75) (end 146.2 109.75) (width 0.4) (layer F.Cu) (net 17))
 (segment (start 147.025 104.265) (end 147.025 107.475) (width 0.4) (layer F.Cu) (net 17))
 (segment (start 147.025 101.925) (end 147.025 104.265) (width 0.4) (layer F.Cu) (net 17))
 (segment (start 145.5 104.25) (end 144.55 104.25) (width 0.15) (layer F.Cu) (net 17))
 (segment (start 147.025 104.265) (end 147.01 104.25) (width 0.15) (layer F.Cu) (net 17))
 (segment (start 147.01 104.25) (end 145.5 104.25) (width 0.15) (layer F.Cu) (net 17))
 (segment (start 144.64 101.4) (end 146.5 101.4) (width 0.4) (layer B.Cu) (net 17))
 (via (at 144.64 101.4) (size 0.6) (drill 0.4) (layers F.Cu B.Cu) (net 17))
 (segment (start 144.64 102.16) (end 144.55 102.25) (width 0.15) (layer F.Cu) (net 17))
 (segment (start 144.64 101.4) (end 144.64 102.16) (width 0.4) (layer F.Cu) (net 17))
 (segment (start 144.02 100.78) (end 144.64 101.4) (width 0.4) (layer F.Cu) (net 17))
 (segment (start 144.02 95.92501) (end 144.02 100.78) (width 0.4) (layer F.Cu) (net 17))
 (segment (start 141.85 109.95) (end 141.005 109.95) (width 0.15) (layer F.Cu) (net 29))
 (segment (start 141.005 109.95) (end 141 109.945) (width 0.15) (layer F.Cu) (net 29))
 (segment (start 143.975 110.25) (end 142.15 110.25) (width 0.15) (layer F.Cu) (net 29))
 (segment (start 142.15 110.25) (end 141.85 109.95) (width 0.15) (layer F.Cu) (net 29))
 (segment (start 143.975 111.25) (end 142.88 111.25) (width 0.15) (layer F.Cu) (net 30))
 (segment (start 141.645 112.485) (end 141 112.485) (width 0.15) (layer F.Cu) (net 30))
 (segment (start 142.88 111.25) (end 141.645 112.485) (width 0.15) (layer F.Cu) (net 30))
 (segment (start 149.725 109.75) (end 149.075 109.75) (width 0.15) (layer F.Cu) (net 12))
 (segment (start 150.35 112.9) (end 150.35 110.375) (width 0.15) (layer F.Cu) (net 12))
 (segment (start 152 113.755) (end 151.205 113.755) (width 0.15) (layer F.Cu) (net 12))
 (segment (start 150.35 110.375) (end 149.725 109.75) (width 0.15) (layer F.Cu) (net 12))
 (segment (start 151.205 113.755) (end 150.35 112.9) (width 0.15) (layer F.Cu) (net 12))
 (segment (start 150.7 110.25) (end 149.7 109.25) (width 0.15) (layer F.Cu) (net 11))
 (segment (start 149.7 109.25) (end 149.075 109.25) (width 0.15) (layer F.Cu) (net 11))
 (segment (start 150.7 111.785) (end 150.7 110.25) (width 0.15) (layer F.Cu) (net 11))
 (segment (start 152 112.485) (end 151.4 112.485) (width 0.15) (layer F.Cu) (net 11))
 (segment (start 151.4 112.485) (end 150.7 111.785) (width 0.15) (layer F.Cu) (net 11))
 (segment (start 151.05 110.062139) (end 149.737861 108.75) (width 0.15) (layer F.Cu) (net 10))
 (segment (start 151.05 110.865) (end 151.05 110.062139) (width 0.15) (layer F.Cu) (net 10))
 (segment (start 149.737861 108.75) (end 149.075 108.75) (width 0.15) (layer F.Cu) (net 10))
 (segment (start 152 111.215) (end 151.4 111.215) (width 0.15) (layer F.Cu) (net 10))
 (segment (start 151.4 111.215) (end 151.05 110.865) (width 0.15) (layer F.Cu) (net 10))
 (segment (start 149.7 108.25) (end 149.075 108.25) (width 0.15) (layer F.Cu) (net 9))
 (segment (start 152 109.945) (end 151.395 109.945) (width 0.15) (layer F.Cu) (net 9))
 (segment (start 151.395 109.945) (end 149.7 108.25) (width 0.15) (layer F.Cu) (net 9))
 (segment (start 151.285 108.675) (end 152 108.675) (width 0.15) (layer F.Cu) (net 8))
 (segment (start 149.025 107.75) (end 150.36 107.75) (width 0.15) (layer F.Cu) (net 8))
 (segment (start 150.36 107.75) (end 151.285 108.675) (width 0.15) (layer F.Cu) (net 8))
 (segment (start 151.845 107.25) (end 149.025 107.25) (width 0.15) (layer F.Cu) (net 7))
 (segment (start 152 107.405) (end 151.845 107.25) (width 0.15) (layer F.Cu) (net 7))
 (segment (start 151.985 106.15) (end 152 106.135) (width 0.15) (layer F.Cu) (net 6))
 (segment (start 150.9 106.15) (end 151.985 106.15) (width 0.15) (layer F.Cu) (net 6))
 (segment (start 149.025 106.75) (end 150.3 106.75) (width 0.15) (layer F.Cu) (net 6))
 (segment (start 150.3 106.75) (end 150.9 106.15) (width 0.15) (layer F.Cu) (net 6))
 (segment (start 151.615 104.865) (end 152 104.865) (width 0.15) (layer F.Cu) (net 5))
 (segment (start 149.025 106.25) (end 150.23 106.25) (width 0.15) (layer F.Cu) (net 5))
 (segment (start 150.23 106.25) (end 151.615 104.865) (width 0.15) (layer F.Cu) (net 5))
 (segment (start 151.26 104.58961) (end 151.26 103.735) (width 0.15) (layer F.Cu) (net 4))
 (segment (start 149.125 105.75) (end 150.09961 105.75) (width 0.15) (layer F.Cu) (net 4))
 (segment (start 150.09961 105.75) (end 151.26 104.58961) (width 0.15) (layer F.Cu) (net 4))
 (segment (start 151.26 102.465) (end 151.26 103.735) (width 0.15) (layer F.Cu) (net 4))
 (segment (start 152 102.325) (end 151.4 102.325) (width 0.15) (layer F.Cu) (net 4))
 (segment (start 151.4 102.325) (end 151.26 102.465) (width 0.15) (layer F.Cu) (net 4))
 (segment (start 151.265 103.595) (end 152 103.595) (width 0.15) (layer F.Cu) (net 4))
 (segment (start 151.26 103.735) (end 151.26 103.6) (width 0.15) (layer F.Cu) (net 4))
 (segment (start 151.26 103.6) (end 151.265 103.595) (width 0.15) (layer F.Cu) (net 4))
 (segment (start 150.96 101.495) (end 151.4 101.055) (width 0.15) (layer F.Cu) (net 3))
 (segment (start 150.96 104.465332) (end 150.96 101.495) (width 0.15) (layer F.Cu) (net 3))
 (segment (start 151.4 101.055) (end 152 101.055) (width 0.15) (layer F.Cu) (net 3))
 (segment (start 149.125 105.25) (end 150.175332 105.25) (width 0.15) (layer F.Cu) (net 3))
 (segment (start 150.175332 105.25) (end 150.96 104.465332) (width 0.15) (layer F.Cu) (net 3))
 (segment (start 150.64 99.275) (end 151.4 98.515) (width 0.15) (layer F.Cu) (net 2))
 (segment (start 151.4 98.515) (end 152 98.515) (width 0.15) (layer F.Cu) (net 2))
 (segment (start 150.64 104.361054) (end 150.64 99.275) (width 0.15) (layer F.Cu) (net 2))
 (segment (start 149.125 104.75) (end 150.251054 104.75) (width 0.15) (layer F.Cu) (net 2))
 (segment (start 150.251054 104.75) (end 150.64 104.361054) (width 0.15) (layer F.Cu) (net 2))
 (segment (start 152 97.245) (end 150.144998 97.245) (width 0.8) (layer F.Cu) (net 1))
 (segment (start 149.8 102.25) (end 150.05 102.25) (width 0.15) (layer F.Cu) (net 1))
 (segment (start 149.025 102.25) (end 149.8 102.25) (width 0.15) (layer F.Cu) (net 1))
 (segment (start 149.8 102.75) (end 150.05 102.75) (width 0.15) (layer F.Cu) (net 1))
 (segment (start 149.025 102.75) (end 149.8 102.75) (width 0.15) (layer F.Cu) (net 1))
 (segment (start 149.025 103.25) (end 150.21 103.25) (width 0.15) (layer F.Cu) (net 1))
 (segment (start 149.025 103.75) (end 150.21 103.75) (width 0.15) (layer F.Cu) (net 1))
 (segment (start 150.15 104.25) (end 150.21 104.19) (width 0.15) (layer F.Cu) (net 1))
 (segment (start 149.025 104.25) (end 150.15 104.25) (width 0.15) (layer F.Cu) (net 1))
 (segment (start 150.01 97.1) (end 150.01 101.5) (width 0.8) (layer F.Cu) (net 1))
 (segment (start 150.19 101.68) (end 150.19 104.19) (width 0.4) (layer F.Cu) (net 1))
 (segment (start 150.01 101.5) (end 150.19 101.68) (width 0.4) (layer F.Cu) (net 1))
 (segment (start 143.325 97.475) (end 142.95 97.1) (width 0.15) (layer F.Cu) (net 18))
 (segment (start 143.325 102.575) (end 143.325 97.475) (width 0.15) (layer F.Cu) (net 18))
 (segment (start 143.975 102.75) (end 143.5 102.75) (width 0.15) (layer F.Cu) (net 18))
 (segment (start 143.5 102.75) (end 143.325 102.575) (width 0.15) (layer F.Cu) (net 18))
 (segment (start 146.02501 101.89501) (end 145.1 100.97) (width 0.15) (layer F.Cu) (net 19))
 (segment (start 145.1 100.97) (end 145.1 96.7) (width 0.15) (layer F.Cu) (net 19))
 (segment (start 146.02501 103.39999) (end 146.02501 101.89501) (width 0.15) (layer F.Cu) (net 19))
 (segment (start 144.55 103.75) (end 145.675 103.75) (width 0.15) (layer F.Cu) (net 19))
 (segment (start 145.675 103.75) (end 146.02501 103.39999) (width 0.15) (layer F.Cu) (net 19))
 (segment (start 149.75 110.25) (end 150 110.5) (width 0.15) (layer F.Cu) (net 13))
 (segment (start 149.075 110.25) (end 149.75 110.25) (width 0.15) (layer F.Cu) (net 13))
 (segment (start 150 116.2) (end 150 110.5) (width 0.15) (layer F.Cu) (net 13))
 (segment (start 148.45 110.75) (end 147.326442 110.75) (width 0.15) (layer F.Cu) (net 14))
 (segment (start 147.326442 110.75) (end 143 115.076442) (width 0.15) (layer F.Cu) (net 14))
 (segment (start 143 116.2) (end 143 115.076442) (width 0.15) (layer F.Cu) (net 14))
 (segment (start 147.250721 111.25) (end 144.27 114.230721) (width 0.15) (layer F.Cu) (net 15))
 (segment (start 148.45 111.25) (end 147.250721 111.25) (width 0.15) (layer F.Cu) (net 15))
 (segment (start 144.27 116.2) (end 144.27 114.230721) (width 0.15) (layer F.Cu) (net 15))
 (segment (start 148.45 111.75) (end 147.175 111.75) (width 0.15) (layer F.Cu) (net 16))
 (segment (start 147.175 111.75) (end 145.54 113.385) (width 0.15) (layer F.Cu) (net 16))
 (segment (start 145.54 116.2) (end 145.54 113.385) (width 0.15) (layer F.Cu) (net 16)))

